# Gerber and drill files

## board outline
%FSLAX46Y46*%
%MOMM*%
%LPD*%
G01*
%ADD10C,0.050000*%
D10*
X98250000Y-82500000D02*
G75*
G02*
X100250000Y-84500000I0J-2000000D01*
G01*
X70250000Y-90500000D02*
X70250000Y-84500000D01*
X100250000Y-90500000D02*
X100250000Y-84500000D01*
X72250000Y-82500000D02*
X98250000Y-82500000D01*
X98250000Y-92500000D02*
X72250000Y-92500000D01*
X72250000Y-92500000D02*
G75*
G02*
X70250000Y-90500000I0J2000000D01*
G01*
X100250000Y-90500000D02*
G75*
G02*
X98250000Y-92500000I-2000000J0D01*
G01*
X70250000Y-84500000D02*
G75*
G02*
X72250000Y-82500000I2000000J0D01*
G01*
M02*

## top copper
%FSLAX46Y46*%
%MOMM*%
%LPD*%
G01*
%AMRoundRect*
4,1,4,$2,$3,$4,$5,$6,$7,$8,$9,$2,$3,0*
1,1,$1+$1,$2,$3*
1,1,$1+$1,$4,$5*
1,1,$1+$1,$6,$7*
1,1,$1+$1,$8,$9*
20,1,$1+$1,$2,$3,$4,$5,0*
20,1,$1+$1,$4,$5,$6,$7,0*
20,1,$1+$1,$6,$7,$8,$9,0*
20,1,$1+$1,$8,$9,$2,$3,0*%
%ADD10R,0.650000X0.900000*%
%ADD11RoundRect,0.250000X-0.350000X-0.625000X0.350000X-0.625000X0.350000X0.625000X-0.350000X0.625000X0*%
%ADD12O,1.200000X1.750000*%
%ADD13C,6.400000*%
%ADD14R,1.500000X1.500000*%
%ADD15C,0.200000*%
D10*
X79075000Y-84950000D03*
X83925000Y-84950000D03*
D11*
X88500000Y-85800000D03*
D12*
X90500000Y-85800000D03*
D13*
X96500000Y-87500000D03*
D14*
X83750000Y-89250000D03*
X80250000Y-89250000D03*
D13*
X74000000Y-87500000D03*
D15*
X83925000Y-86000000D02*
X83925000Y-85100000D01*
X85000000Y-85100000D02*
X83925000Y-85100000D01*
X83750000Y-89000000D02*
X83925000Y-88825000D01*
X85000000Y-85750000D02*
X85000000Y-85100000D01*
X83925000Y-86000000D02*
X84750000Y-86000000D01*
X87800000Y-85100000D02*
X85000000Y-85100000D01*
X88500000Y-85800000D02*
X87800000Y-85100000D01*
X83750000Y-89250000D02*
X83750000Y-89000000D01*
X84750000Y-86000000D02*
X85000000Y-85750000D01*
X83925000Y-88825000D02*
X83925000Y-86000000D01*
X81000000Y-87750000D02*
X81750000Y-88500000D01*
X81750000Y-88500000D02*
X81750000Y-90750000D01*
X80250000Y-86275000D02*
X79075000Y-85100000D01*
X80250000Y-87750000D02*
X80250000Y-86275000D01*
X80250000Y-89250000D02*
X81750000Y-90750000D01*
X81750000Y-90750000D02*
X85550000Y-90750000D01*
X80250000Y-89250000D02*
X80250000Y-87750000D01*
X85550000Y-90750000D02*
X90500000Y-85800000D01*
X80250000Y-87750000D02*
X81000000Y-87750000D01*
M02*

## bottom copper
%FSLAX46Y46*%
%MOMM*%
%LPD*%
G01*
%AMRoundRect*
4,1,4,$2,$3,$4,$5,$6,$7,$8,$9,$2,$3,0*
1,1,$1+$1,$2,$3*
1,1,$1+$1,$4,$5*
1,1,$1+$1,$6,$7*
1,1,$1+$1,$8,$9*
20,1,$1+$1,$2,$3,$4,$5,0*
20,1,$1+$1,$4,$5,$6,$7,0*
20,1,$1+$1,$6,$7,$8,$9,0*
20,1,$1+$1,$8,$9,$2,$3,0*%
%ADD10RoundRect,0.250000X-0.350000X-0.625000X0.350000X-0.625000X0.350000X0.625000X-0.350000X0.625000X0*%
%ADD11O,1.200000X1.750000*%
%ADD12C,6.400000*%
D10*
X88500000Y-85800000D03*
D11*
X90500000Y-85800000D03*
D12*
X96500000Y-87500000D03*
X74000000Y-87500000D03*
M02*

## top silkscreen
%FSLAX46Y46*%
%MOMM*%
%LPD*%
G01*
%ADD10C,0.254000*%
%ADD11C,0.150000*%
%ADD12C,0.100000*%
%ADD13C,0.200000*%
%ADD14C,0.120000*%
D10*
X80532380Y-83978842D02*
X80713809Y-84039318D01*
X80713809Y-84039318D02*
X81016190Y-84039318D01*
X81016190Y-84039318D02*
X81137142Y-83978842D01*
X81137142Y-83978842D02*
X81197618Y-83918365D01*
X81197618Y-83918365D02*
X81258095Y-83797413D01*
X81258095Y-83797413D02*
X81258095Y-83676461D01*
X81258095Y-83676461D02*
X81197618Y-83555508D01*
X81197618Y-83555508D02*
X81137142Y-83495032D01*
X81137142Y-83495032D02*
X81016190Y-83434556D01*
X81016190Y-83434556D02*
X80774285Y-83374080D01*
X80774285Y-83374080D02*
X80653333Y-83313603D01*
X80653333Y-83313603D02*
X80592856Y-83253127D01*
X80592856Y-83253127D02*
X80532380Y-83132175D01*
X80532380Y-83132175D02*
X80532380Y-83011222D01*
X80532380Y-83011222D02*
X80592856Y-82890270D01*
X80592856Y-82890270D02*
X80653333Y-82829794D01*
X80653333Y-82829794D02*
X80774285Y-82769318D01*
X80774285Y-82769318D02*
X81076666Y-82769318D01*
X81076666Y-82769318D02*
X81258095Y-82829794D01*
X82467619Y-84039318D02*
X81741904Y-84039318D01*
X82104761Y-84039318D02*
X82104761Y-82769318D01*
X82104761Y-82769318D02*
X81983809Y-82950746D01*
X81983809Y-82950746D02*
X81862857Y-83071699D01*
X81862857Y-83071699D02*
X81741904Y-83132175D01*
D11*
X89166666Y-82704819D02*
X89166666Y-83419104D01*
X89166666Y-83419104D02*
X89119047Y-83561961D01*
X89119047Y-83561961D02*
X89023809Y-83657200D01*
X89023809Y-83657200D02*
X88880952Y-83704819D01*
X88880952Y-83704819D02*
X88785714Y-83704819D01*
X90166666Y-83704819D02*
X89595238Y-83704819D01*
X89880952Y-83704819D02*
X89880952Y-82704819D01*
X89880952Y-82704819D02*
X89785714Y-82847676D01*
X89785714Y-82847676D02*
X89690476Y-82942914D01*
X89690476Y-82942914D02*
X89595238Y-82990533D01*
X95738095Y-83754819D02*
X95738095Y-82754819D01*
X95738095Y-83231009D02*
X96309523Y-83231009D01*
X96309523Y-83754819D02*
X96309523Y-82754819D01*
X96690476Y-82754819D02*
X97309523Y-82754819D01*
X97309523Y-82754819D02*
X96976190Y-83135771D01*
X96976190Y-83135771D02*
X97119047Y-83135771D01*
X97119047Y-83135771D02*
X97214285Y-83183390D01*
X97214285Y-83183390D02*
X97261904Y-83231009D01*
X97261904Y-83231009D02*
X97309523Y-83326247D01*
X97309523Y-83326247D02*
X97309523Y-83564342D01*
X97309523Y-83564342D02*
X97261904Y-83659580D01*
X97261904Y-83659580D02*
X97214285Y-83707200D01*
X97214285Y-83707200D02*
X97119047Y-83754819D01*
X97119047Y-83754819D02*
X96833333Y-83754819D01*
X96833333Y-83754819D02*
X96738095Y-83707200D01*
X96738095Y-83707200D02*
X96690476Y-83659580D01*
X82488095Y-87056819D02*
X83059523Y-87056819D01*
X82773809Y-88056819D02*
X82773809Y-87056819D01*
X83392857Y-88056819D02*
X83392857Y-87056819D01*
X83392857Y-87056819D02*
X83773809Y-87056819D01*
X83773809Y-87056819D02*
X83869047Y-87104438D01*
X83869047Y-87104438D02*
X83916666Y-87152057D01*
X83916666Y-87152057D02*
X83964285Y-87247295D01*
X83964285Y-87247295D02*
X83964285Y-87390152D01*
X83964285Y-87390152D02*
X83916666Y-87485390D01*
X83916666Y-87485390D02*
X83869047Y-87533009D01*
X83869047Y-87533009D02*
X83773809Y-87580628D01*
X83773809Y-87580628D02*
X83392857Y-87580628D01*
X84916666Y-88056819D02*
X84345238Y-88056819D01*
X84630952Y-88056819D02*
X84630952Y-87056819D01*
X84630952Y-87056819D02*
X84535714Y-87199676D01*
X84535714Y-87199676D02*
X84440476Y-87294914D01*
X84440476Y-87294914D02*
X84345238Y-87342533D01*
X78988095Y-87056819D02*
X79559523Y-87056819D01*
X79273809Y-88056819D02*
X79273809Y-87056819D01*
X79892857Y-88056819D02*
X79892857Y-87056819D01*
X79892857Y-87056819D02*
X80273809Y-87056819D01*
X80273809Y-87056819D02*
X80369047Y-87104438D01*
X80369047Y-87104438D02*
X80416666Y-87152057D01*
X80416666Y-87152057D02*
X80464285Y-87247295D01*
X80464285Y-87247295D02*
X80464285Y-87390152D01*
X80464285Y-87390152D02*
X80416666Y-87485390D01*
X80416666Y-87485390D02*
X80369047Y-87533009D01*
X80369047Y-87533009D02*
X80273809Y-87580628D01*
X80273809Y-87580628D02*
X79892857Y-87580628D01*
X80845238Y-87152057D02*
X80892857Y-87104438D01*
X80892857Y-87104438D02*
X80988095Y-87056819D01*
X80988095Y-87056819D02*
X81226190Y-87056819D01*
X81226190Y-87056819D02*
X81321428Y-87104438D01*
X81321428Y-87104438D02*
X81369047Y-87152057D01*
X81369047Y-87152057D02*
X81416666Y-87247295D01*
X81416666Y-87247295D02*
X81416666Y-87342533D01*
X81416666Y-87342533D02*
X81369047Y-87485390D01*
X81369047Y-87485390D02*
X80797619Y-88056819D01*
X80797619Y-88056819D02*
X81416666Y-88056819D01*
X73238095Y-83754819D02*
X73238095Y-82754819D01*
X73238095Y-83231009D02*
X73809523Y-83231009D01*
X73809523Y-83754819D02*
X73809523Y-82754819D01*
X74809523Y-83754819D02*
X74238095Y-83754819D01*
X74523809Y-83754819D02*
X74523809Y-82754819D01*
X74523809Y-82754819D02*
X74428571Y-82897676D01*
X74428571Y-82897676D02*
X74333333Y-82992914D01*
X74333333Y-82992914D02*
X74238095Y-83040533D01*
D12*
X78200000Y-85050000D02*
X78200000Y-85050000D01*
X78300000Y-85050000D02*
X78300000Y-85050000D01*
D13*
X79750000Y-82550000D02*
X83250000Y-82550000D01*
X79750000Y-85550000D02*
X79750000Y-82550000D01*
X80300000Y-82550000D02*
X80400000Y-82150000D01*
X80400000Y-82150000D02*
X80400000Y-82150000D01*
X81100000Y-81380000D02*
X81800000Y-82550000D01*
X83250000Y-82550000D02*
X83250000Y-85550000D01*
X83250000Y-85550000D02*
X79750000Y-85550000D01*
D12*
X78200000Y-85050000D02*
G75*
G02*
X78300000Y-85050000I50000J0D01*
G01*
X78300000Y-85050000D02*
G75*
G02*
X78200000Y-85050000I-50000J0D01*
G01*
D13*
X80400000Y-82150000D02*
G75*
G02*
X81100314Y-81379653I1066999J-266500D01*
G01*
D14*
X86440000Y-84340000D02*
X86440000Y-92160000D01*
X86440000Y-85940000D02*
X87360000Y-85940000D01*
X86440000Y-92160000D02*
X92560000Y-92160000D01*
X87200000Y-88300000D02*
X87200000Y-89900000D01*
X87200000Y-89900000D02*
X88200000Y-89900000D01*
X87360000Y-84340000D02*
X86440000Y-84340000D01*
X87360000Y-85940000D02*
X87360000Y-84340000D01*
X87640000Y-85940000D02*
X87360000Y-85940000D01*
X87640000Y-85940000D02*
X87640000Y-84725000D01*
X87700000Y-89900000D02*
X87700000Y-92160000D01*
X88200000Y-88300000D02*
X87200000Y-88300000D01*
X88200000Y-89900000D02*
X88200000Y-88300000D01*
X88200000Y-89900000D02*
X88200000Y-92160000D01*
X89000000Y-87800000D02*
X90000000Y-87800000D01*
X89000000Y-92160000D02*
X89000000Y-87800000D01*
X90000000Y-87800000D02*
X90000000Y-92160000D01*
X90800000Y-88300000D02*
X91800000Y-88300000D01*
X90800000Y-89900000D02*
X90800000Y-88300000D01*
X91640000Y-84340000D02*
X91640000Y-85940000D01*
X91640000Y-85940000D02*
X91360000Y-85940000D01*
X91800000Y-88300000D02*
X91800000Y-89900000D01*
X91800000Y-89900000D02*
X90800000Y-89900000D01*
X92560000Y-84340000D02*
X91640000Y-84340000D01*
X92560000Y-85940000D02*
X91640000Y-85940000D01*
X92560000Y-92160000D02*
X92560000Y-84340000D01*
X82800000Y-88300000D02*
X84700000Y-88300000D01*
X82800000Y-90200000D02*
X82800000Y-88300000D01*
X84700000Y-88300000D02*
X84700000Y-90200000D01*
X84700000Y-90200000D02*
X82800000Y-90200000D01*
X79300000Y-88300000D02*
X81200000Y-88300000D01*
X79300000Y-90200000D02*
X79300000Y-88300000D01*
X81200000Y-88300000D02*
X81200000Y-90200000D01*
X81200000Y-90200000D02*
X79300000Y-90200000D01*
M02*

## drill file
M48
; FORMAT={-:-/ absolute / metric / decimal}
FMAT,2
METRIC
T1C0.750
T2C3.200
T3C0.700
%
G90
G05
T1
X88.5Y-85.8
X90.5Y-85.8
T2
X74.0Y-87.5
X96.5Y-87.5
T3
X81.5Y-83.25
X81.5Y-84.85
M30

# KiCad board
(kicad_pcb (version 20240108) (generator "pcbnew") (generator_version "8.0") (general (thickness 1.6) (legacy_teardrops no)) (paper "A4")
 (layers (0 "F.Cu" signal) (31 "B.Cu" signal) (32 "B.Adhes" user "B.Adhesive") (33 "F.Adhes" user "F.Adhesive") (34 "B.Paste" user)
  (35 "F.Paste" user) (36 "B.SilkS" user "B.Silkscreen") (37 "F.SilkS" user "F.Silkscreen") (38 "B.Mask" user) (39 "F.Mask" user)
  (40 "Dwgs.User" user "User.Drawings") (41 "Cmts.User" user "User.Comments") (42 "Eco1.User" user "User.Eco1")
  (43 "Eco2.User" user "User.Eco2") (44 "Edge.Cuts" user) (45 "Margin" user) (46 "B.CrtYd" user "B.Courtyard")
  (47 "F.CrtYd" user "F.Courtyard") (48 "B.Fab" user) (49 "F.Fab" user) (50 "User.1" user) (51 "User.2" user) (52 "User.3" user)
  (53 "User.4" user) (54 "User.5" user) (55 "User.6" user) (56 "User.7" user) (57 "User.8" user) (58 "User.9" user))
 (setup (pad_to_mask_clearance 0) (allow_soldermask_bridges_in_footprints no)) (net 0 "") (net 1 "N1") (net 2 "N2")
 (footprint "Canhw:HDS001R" (layer "F.Cu") (at 81.5 84.05)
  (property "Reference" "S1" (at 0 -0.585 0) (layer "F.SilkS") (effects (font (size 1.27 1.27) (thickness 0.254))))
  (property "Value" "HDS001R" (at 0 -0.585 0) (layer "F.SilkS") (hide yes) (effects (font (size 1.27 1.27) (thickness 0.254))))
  (fp_line (start -3.3 1) (end -3.3 1) (stroke (width 0.1) (type solid)) (layer "F.SilkS"))
  (fp_line (start -3.2 1) (end -3.2 1) (stroke (width 0.1) (type solid)) (layer "F.SilkS"))
  (fp_line (start -1.75 -1.5) (end 1.75 -1.5) (stroke (width 0.2) (type solid)) (layer "F.SilkS"))
  (fp_line (start -1.75 1.5) (end -1.75 -1.5) (stroke (width 0.2) (type solid)) (layer "F.SilkS"))
  (fp_line (start -1.2 -1.5) (end -1.1 -1.9) (stroke (width 0.2) (type solid)) (layer "F.SilkS"))
  (fp_line (start -1.1 -1.9) (end -1.1 -1.9) (stroke (width 0.2) (type solid)) (layer "F.SilkS"))
  (fp_line (start -0.4 -2.67) (end 0.3 -1.5) (stroke (width 0.2) (type solid)) (layer "F.SilkS"))
  (fp_line (start 1.75 -1.5) (end 1.75 1.5) (stroke (width 0.2) (type solid)) (layer "F.SilkS"))
  (fp_line (start 1.75 1.5) (end -1.75 1.5) (stroke (width 0.2) (type solid)) (layer "F.SilkS"))
  (fp_arc (start -3.3 1) (mid -3.25 0.95) (end -3.2 1) (stroke (width 0.1) (type solid)) (layer "F.SilkS"))
  (fp_arc (start -3.2 1) (mid -3.25 1.05) (end -3.3 1) (stroke (width 0.1) (type solid)) (layer "F.SilkS"))
  (fp_arc (start -1.1 -1.9) (mid -0.846771 -2.373289) (end -0.399686 -2.670347) (stroke (width 0.2) (type solid)) (layer "F.SilkS"))
  (pad "" np_thru_hole circle (at 0 -0.8) (size 0.7 0.7) (drill 0.7) (layers "*.Cu" "*.Mask"))
  (pad "" np_thru_hole circle (at 0 0.8) (size 0.7 0.7) (drill 0.7) (layers "*.Cu" "*.Mask"))
  (pad "A1" smd rect (at -2.425 0.9) (size 0.65 0.9) (layers "F.Cu" "F.Paste" "F.Mask") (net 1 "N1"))
  (pad "B1" smd rect (at 2.425 0.9) (size 0.65 0.9) (layers "F.Cu" "F.Paste" "F.Mask") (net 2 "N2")))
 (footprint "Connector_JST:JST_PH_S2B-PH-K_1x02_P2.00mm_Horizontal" (layer "F.Cu") (at 88.5 85.8)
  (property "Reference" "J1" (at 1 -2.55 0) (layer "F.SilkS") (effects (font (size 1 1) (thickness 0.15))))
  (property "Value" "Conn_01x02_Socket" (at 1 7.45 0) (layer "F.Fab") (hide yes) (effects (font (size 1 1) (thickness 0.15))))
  (fp_line (start -2.06 -1.46) (end -2.06 6.36) (stroke (width 0.12) (type solid)) (layer "F.SilkS"))
  (fp_line (start -2.06 0.14) (end -1.14 0.14) (stroke (width 0.12) (type solid)) (layer "F.SilkS"))
  (fp_line (start -2.06 6.36) (end 4.06 6.36) (stroke (width 0.12) (type solid)) (layer "F.SilkS"))
  (fp_line (start -1.3 2.5) (end -1.3 4.1) (stroke (width 0.12) (type solid)) (layer "F.SilkS"))
  (fp_line (start -1.3 4.1) (end -0.3 4.1) (stroke (width 0.12) (type solid)) (layer "F.SilkS"))
  (fp_line (start -1.14 -1.46) (end -2.06 -1.46) (stroke (width 0.12) (type solid)) (layer "F.SilkS"))
  (fp_line (start -1.14 0.14) (end -1.14 -1.46) (stroke (width 0.12) (type solid)) (layer "F.SilkS"))
  (fp_line (start -0.86 0.14) (end -1.14 0.14) (stroke (width 0.12) (type solid)) (layer "F.SilkS"))
  (fp_line (start -0.86 0.14) (end -0.86 -1.075) (stroke (width 0.12) (type solid)) (layer "F.SilkS"))
  (fp_line (start -0.8 4.1) (end -0.8 6.36) (stroke (width 0.12) (type solid)) (layer "F.SilkS"))
  (fp_line (start -0.3 2.5) (end -1.3 2.5) (stroke (width 0.12) (type solid)) (layer "F.SilkS"))
  (fp_line (start -0.3 4.1) (end -0.3 2.5) (stroke (width 0.12) (type solid)) (layer "F.SilkS"))
  (fp_line (start -0.3 4.1) (end -0.3 6.36) (stroke (width 0.12) (type solid)) (layer "F.SilkS"))
  (fp_line (start 0.5 2) (end 1.5 2) (stroke (width 0.12) (type solid)) (layer "F.SilkS"))
  (fp_line (start 0.5 6.36) (end 0.5 2) (stroke (width 0.12) (type solid)) (layer "F.SilkS"))
  (fp_line (start 1.5 2) (end 1.5 6.36) (stroke (width 0.12) (type solid)) (layer "F.SilkS"))
  (fp_line (start 2.3 2.5) (end 3.3 2.5) (stroke (width 0.12) (type solid)) (layer "F.SilkS"))
  (fp_line (start 2.3 4.1) (end 2.3 2.5) (stroke (width 0.12) (type solid)) (layer "F.SilkS"))
  (fp_line (start 3.14 -1.46) (end 3.14 0.14) (stroke (width 0.12) (type solid)) (layer "F.SilkS"))
  (fp_line (start 3.14 0.14) (end 2.86 0.14) (stroke (width 0.12) (type solid)) (layer "F.SilkS"))
  (fp_line (start 3.3 2.5) (end 3.3 4.1) (stroke (width 0.12) (type solid)) (layer "F.SilkS"))
  (fp_line (start 3.3 4.1) (end 2.3 4.1) (stroke (width 0.12) (type solid)) (layer "F.SilkS"))
  (fp_line (start 4.06 -1.46) (end 3.14 -1.46) (stroke (width 0.12) (type solid)) (layer "F.SilkS"))
  (fp_line (start 4.06 0.14) (end 3.14 0.14) (stroke (width 0.12) (type solid)) (layer "F.SilkS"))
  (fp_line (start 4.06 6.36) (end 4.06 -1.46) (stroke (width 0.12) (type solid)) (layer "F.SilkS"))
  (pad "1" thru_hole roundrect (at 0 0) (size 1.2 1.75) (drill 0.75) (layers "*.Cu" "*.Mask") (remove_unused_layers no)
   (roundrect_rratio 0.208333) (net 2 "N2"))
  (pad "2" thru_hole oval (at 2 0) (size 1.2 1.75) (drill 0.75) (layers "*.Cu" "*.Mask") (remove_unused_layers no) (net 1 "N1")))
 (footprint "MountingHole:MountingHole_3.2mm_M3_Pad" (layer "F.Cu") (at 96.5 87.5)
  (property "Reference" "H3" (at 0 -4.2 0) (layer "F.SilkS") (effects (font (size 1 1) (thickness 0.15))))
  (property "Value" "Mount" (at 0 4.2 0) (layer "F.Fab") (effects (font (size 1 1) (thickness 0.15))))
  (pad "1" thru_hole circle (at 0 0) (size 6.4 6.4) (drill 3.2) (layers "*.Cu" "*.Mask") (remove_unused_layers no)))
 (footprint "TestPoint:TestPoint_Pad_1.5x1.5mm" (layer "F.Cu") (at 83.75 89.25)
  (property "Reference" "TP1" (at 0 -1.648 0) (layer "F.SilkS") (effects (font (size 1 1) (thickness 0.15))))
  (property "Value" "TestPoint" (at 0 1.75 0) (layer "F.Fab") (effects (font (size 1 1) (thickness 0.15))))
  (fp_line (start -0.95 -0.95) (end 0.95 -0.95) (stroke (width 0.12) (type solid)) (layer "F.SilkS"))
  (fp_line (start -0.95 0.95) (end -0.95 -0.95) (stroke (width 0.12) (type solid)) (layer "F.SilkS"))
  (fp_line (start 0.95 -0.95) (end 0.95 0.95) (stroke (width 0.12) (type solid)) (layer "F.SilkS"))
  (fp_line (start 0.95 0.95) (end -0.95 0.95) (stroke (width 0.12) (type solid)) (layer "F.SilkS"))
  (pad "1" smd rect (at 0 0) (size 1.5 1.5) (layers "F.Cu" "F.Mask") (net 2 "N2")))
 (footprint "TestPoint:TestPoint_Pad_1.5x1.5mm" (layer "F.Cu") (at 80.25 89.25)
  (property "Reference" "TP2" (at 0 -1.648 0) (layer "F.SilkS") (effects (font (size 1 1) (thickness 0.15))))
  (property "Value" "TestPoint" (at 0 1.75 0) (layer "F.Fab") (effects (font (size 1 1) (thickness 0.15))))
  (fp_line (start -0.95 -0.95) (end 0.95 -0.95) (stroke (width 0.12) (type solid)) (layer "F.SilkS"))
  (fp_line (start -0.95 0.95) (end -0.95 -0.95) (stroke (width 0.12) (type solid)) (layer "F.SilkS"))
  (fp_line (start 0.95 -0.95) (end 0.95 0.95) (stroke (width 0.12) (type solid)) (layer "F.SilkS"))
  (fp_line (start 0.95 0.95) (end -0.95 0.95) (stroke (width 0.12) (type solid)) (layer "F.SilkS"))
  (pad "1" smd rect (at 0 0) (size 1.5 1.5) (layers "F.Cu" "F.Mask") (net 1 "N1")))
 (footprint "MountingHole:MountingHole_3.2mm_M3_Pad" (layer "F.Cu") (at 74 87.5)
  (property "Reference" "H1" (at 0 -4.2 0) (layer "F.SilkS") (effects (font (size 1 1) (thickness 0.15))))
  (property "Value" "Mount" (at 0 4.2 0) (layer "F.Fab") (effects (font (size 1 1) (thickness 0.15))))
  (pad "1" thru_hole circle (at 0 0) (size 6.4 6.4) (drill 3.2) (layers "*.Cu" "*.Mask") (remove_unused_layers no)))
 (gr_arc (start 98.25 82.5) (mid 99.664214 83.085786) (end 100.25 84.5) (stroke (width 0.05) (type default)) (layer "Edge.Cuts"))
 (gr_line (start 70.25 90.5) (end 70.25 84.5) (stroke (width 0.05) (type default)) (layer "Edge.Cuts"))
 (gr_line (start 100.25 90.5) (end 100.25 84.5) (stroke (width 0.05) (type default)) (layer "Edge.Cuts"))
 (gr_line (start 72.25 82.5) (end 98.25 82.5) (stroke (width 0.05) (type default)) (layer "Edge.Cuts"))
 (gr_line (start 98.25 92.5) (end 72.25 92.5) (stroke (width 0.05) (type default)) (layer "Edge.Cuts"))
 (gr_arc (start 72.25 92.5) (mid 70.835786 91.914214) (end 70.25 90.5) (stroke (width 0.05) (type default)) (layer "Edge.Cuts"))
 (gr_arc (start 100.25 90.5) (mid 99.664214 91.914214) (end 98.25 92.5) (stroke (width 0.05) (type default)) (layer "Edge.Cuts"))
 (gr_arc (start 70.25 84.5) (mid 70.835786 83.085786) (end 72.25 82.5) (stroke (width 0.05) (type default)) (layer "Edge.Cuts"))
 (segment (start 83.925 86) (end 83.925 85.1) (width 0.2) (layer "F.Cu") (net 2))
 (segment (start 85 85.1) (end 83.925 85.1) (width 0.2) (layer "F.Cu") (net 2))
 (segment (start 83.75 89) (end 83.925 88.825) (width 0.2) (layer "F.Cu") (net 2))
 (segment (start 85 85.75) (end 85 85.1) (width 0.2) (layer "F.Cu") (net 2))
 (segment (start 83.925 86) (end 84.75 86) (width 0.2) (layer "F.Cu") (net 2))
 (segment (start 87.8 85.1) (end 85 85.1) (width 0.2) (layer "F.Cu") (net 2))
 (segment (start 88.5 85.8) (end 87.8 85.1) (width 0.2) (layer "F.Cu") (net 2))
 (segment (start 83.75 89.25) (end 83.75 89) (width 0.2) (layer "F.Cu") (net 2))
 (segment (start 84.75 86) (end 85 85.75) (width 0.2) (layer "F.Cu") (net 2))
 (segment (start 83.925 88.825) (end 83.925 86) (width 0.2) (layer "F.Cu") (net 2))
 (segment (start 81 87.75) (end 81.75 88.5) (width 0.2) (layer "F.Cu") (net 1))
 (segment (start 81.75 88.5) (end 81.75 90.75) (width 0.2) (layer "F.Cu") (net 1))
 (segment (start 80.25 86.275) (end 79.075 85.1) (width 0.2) (layer "F.Cu") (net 1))
 (segment (start 80.25 87.75) (end 80.25 86.275) (width 0.2) (layer "F.Cu") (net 1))
 (segment (start 80.25 89.25) (end 81.75 90.75) (width 0.2) (layer "F.Cu") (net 1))
 (segment (start 81.75 90.75) (end 85.55 90.75) (width 0.2) (layer "F.Cu") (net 1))
 (segment (start 80.25 89.25) (end 80.25 87.75) (width 0.2) (layer "F.Cu") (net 1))
 (segment (start 85.55 90.75) (end 90.5 85.8) (width 0.2) (layer "F.Cu") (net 1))
 (segment (start 80.25 87.75) (end 81 87.75) (width 0.2) (layer "F.Cu") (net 1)))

